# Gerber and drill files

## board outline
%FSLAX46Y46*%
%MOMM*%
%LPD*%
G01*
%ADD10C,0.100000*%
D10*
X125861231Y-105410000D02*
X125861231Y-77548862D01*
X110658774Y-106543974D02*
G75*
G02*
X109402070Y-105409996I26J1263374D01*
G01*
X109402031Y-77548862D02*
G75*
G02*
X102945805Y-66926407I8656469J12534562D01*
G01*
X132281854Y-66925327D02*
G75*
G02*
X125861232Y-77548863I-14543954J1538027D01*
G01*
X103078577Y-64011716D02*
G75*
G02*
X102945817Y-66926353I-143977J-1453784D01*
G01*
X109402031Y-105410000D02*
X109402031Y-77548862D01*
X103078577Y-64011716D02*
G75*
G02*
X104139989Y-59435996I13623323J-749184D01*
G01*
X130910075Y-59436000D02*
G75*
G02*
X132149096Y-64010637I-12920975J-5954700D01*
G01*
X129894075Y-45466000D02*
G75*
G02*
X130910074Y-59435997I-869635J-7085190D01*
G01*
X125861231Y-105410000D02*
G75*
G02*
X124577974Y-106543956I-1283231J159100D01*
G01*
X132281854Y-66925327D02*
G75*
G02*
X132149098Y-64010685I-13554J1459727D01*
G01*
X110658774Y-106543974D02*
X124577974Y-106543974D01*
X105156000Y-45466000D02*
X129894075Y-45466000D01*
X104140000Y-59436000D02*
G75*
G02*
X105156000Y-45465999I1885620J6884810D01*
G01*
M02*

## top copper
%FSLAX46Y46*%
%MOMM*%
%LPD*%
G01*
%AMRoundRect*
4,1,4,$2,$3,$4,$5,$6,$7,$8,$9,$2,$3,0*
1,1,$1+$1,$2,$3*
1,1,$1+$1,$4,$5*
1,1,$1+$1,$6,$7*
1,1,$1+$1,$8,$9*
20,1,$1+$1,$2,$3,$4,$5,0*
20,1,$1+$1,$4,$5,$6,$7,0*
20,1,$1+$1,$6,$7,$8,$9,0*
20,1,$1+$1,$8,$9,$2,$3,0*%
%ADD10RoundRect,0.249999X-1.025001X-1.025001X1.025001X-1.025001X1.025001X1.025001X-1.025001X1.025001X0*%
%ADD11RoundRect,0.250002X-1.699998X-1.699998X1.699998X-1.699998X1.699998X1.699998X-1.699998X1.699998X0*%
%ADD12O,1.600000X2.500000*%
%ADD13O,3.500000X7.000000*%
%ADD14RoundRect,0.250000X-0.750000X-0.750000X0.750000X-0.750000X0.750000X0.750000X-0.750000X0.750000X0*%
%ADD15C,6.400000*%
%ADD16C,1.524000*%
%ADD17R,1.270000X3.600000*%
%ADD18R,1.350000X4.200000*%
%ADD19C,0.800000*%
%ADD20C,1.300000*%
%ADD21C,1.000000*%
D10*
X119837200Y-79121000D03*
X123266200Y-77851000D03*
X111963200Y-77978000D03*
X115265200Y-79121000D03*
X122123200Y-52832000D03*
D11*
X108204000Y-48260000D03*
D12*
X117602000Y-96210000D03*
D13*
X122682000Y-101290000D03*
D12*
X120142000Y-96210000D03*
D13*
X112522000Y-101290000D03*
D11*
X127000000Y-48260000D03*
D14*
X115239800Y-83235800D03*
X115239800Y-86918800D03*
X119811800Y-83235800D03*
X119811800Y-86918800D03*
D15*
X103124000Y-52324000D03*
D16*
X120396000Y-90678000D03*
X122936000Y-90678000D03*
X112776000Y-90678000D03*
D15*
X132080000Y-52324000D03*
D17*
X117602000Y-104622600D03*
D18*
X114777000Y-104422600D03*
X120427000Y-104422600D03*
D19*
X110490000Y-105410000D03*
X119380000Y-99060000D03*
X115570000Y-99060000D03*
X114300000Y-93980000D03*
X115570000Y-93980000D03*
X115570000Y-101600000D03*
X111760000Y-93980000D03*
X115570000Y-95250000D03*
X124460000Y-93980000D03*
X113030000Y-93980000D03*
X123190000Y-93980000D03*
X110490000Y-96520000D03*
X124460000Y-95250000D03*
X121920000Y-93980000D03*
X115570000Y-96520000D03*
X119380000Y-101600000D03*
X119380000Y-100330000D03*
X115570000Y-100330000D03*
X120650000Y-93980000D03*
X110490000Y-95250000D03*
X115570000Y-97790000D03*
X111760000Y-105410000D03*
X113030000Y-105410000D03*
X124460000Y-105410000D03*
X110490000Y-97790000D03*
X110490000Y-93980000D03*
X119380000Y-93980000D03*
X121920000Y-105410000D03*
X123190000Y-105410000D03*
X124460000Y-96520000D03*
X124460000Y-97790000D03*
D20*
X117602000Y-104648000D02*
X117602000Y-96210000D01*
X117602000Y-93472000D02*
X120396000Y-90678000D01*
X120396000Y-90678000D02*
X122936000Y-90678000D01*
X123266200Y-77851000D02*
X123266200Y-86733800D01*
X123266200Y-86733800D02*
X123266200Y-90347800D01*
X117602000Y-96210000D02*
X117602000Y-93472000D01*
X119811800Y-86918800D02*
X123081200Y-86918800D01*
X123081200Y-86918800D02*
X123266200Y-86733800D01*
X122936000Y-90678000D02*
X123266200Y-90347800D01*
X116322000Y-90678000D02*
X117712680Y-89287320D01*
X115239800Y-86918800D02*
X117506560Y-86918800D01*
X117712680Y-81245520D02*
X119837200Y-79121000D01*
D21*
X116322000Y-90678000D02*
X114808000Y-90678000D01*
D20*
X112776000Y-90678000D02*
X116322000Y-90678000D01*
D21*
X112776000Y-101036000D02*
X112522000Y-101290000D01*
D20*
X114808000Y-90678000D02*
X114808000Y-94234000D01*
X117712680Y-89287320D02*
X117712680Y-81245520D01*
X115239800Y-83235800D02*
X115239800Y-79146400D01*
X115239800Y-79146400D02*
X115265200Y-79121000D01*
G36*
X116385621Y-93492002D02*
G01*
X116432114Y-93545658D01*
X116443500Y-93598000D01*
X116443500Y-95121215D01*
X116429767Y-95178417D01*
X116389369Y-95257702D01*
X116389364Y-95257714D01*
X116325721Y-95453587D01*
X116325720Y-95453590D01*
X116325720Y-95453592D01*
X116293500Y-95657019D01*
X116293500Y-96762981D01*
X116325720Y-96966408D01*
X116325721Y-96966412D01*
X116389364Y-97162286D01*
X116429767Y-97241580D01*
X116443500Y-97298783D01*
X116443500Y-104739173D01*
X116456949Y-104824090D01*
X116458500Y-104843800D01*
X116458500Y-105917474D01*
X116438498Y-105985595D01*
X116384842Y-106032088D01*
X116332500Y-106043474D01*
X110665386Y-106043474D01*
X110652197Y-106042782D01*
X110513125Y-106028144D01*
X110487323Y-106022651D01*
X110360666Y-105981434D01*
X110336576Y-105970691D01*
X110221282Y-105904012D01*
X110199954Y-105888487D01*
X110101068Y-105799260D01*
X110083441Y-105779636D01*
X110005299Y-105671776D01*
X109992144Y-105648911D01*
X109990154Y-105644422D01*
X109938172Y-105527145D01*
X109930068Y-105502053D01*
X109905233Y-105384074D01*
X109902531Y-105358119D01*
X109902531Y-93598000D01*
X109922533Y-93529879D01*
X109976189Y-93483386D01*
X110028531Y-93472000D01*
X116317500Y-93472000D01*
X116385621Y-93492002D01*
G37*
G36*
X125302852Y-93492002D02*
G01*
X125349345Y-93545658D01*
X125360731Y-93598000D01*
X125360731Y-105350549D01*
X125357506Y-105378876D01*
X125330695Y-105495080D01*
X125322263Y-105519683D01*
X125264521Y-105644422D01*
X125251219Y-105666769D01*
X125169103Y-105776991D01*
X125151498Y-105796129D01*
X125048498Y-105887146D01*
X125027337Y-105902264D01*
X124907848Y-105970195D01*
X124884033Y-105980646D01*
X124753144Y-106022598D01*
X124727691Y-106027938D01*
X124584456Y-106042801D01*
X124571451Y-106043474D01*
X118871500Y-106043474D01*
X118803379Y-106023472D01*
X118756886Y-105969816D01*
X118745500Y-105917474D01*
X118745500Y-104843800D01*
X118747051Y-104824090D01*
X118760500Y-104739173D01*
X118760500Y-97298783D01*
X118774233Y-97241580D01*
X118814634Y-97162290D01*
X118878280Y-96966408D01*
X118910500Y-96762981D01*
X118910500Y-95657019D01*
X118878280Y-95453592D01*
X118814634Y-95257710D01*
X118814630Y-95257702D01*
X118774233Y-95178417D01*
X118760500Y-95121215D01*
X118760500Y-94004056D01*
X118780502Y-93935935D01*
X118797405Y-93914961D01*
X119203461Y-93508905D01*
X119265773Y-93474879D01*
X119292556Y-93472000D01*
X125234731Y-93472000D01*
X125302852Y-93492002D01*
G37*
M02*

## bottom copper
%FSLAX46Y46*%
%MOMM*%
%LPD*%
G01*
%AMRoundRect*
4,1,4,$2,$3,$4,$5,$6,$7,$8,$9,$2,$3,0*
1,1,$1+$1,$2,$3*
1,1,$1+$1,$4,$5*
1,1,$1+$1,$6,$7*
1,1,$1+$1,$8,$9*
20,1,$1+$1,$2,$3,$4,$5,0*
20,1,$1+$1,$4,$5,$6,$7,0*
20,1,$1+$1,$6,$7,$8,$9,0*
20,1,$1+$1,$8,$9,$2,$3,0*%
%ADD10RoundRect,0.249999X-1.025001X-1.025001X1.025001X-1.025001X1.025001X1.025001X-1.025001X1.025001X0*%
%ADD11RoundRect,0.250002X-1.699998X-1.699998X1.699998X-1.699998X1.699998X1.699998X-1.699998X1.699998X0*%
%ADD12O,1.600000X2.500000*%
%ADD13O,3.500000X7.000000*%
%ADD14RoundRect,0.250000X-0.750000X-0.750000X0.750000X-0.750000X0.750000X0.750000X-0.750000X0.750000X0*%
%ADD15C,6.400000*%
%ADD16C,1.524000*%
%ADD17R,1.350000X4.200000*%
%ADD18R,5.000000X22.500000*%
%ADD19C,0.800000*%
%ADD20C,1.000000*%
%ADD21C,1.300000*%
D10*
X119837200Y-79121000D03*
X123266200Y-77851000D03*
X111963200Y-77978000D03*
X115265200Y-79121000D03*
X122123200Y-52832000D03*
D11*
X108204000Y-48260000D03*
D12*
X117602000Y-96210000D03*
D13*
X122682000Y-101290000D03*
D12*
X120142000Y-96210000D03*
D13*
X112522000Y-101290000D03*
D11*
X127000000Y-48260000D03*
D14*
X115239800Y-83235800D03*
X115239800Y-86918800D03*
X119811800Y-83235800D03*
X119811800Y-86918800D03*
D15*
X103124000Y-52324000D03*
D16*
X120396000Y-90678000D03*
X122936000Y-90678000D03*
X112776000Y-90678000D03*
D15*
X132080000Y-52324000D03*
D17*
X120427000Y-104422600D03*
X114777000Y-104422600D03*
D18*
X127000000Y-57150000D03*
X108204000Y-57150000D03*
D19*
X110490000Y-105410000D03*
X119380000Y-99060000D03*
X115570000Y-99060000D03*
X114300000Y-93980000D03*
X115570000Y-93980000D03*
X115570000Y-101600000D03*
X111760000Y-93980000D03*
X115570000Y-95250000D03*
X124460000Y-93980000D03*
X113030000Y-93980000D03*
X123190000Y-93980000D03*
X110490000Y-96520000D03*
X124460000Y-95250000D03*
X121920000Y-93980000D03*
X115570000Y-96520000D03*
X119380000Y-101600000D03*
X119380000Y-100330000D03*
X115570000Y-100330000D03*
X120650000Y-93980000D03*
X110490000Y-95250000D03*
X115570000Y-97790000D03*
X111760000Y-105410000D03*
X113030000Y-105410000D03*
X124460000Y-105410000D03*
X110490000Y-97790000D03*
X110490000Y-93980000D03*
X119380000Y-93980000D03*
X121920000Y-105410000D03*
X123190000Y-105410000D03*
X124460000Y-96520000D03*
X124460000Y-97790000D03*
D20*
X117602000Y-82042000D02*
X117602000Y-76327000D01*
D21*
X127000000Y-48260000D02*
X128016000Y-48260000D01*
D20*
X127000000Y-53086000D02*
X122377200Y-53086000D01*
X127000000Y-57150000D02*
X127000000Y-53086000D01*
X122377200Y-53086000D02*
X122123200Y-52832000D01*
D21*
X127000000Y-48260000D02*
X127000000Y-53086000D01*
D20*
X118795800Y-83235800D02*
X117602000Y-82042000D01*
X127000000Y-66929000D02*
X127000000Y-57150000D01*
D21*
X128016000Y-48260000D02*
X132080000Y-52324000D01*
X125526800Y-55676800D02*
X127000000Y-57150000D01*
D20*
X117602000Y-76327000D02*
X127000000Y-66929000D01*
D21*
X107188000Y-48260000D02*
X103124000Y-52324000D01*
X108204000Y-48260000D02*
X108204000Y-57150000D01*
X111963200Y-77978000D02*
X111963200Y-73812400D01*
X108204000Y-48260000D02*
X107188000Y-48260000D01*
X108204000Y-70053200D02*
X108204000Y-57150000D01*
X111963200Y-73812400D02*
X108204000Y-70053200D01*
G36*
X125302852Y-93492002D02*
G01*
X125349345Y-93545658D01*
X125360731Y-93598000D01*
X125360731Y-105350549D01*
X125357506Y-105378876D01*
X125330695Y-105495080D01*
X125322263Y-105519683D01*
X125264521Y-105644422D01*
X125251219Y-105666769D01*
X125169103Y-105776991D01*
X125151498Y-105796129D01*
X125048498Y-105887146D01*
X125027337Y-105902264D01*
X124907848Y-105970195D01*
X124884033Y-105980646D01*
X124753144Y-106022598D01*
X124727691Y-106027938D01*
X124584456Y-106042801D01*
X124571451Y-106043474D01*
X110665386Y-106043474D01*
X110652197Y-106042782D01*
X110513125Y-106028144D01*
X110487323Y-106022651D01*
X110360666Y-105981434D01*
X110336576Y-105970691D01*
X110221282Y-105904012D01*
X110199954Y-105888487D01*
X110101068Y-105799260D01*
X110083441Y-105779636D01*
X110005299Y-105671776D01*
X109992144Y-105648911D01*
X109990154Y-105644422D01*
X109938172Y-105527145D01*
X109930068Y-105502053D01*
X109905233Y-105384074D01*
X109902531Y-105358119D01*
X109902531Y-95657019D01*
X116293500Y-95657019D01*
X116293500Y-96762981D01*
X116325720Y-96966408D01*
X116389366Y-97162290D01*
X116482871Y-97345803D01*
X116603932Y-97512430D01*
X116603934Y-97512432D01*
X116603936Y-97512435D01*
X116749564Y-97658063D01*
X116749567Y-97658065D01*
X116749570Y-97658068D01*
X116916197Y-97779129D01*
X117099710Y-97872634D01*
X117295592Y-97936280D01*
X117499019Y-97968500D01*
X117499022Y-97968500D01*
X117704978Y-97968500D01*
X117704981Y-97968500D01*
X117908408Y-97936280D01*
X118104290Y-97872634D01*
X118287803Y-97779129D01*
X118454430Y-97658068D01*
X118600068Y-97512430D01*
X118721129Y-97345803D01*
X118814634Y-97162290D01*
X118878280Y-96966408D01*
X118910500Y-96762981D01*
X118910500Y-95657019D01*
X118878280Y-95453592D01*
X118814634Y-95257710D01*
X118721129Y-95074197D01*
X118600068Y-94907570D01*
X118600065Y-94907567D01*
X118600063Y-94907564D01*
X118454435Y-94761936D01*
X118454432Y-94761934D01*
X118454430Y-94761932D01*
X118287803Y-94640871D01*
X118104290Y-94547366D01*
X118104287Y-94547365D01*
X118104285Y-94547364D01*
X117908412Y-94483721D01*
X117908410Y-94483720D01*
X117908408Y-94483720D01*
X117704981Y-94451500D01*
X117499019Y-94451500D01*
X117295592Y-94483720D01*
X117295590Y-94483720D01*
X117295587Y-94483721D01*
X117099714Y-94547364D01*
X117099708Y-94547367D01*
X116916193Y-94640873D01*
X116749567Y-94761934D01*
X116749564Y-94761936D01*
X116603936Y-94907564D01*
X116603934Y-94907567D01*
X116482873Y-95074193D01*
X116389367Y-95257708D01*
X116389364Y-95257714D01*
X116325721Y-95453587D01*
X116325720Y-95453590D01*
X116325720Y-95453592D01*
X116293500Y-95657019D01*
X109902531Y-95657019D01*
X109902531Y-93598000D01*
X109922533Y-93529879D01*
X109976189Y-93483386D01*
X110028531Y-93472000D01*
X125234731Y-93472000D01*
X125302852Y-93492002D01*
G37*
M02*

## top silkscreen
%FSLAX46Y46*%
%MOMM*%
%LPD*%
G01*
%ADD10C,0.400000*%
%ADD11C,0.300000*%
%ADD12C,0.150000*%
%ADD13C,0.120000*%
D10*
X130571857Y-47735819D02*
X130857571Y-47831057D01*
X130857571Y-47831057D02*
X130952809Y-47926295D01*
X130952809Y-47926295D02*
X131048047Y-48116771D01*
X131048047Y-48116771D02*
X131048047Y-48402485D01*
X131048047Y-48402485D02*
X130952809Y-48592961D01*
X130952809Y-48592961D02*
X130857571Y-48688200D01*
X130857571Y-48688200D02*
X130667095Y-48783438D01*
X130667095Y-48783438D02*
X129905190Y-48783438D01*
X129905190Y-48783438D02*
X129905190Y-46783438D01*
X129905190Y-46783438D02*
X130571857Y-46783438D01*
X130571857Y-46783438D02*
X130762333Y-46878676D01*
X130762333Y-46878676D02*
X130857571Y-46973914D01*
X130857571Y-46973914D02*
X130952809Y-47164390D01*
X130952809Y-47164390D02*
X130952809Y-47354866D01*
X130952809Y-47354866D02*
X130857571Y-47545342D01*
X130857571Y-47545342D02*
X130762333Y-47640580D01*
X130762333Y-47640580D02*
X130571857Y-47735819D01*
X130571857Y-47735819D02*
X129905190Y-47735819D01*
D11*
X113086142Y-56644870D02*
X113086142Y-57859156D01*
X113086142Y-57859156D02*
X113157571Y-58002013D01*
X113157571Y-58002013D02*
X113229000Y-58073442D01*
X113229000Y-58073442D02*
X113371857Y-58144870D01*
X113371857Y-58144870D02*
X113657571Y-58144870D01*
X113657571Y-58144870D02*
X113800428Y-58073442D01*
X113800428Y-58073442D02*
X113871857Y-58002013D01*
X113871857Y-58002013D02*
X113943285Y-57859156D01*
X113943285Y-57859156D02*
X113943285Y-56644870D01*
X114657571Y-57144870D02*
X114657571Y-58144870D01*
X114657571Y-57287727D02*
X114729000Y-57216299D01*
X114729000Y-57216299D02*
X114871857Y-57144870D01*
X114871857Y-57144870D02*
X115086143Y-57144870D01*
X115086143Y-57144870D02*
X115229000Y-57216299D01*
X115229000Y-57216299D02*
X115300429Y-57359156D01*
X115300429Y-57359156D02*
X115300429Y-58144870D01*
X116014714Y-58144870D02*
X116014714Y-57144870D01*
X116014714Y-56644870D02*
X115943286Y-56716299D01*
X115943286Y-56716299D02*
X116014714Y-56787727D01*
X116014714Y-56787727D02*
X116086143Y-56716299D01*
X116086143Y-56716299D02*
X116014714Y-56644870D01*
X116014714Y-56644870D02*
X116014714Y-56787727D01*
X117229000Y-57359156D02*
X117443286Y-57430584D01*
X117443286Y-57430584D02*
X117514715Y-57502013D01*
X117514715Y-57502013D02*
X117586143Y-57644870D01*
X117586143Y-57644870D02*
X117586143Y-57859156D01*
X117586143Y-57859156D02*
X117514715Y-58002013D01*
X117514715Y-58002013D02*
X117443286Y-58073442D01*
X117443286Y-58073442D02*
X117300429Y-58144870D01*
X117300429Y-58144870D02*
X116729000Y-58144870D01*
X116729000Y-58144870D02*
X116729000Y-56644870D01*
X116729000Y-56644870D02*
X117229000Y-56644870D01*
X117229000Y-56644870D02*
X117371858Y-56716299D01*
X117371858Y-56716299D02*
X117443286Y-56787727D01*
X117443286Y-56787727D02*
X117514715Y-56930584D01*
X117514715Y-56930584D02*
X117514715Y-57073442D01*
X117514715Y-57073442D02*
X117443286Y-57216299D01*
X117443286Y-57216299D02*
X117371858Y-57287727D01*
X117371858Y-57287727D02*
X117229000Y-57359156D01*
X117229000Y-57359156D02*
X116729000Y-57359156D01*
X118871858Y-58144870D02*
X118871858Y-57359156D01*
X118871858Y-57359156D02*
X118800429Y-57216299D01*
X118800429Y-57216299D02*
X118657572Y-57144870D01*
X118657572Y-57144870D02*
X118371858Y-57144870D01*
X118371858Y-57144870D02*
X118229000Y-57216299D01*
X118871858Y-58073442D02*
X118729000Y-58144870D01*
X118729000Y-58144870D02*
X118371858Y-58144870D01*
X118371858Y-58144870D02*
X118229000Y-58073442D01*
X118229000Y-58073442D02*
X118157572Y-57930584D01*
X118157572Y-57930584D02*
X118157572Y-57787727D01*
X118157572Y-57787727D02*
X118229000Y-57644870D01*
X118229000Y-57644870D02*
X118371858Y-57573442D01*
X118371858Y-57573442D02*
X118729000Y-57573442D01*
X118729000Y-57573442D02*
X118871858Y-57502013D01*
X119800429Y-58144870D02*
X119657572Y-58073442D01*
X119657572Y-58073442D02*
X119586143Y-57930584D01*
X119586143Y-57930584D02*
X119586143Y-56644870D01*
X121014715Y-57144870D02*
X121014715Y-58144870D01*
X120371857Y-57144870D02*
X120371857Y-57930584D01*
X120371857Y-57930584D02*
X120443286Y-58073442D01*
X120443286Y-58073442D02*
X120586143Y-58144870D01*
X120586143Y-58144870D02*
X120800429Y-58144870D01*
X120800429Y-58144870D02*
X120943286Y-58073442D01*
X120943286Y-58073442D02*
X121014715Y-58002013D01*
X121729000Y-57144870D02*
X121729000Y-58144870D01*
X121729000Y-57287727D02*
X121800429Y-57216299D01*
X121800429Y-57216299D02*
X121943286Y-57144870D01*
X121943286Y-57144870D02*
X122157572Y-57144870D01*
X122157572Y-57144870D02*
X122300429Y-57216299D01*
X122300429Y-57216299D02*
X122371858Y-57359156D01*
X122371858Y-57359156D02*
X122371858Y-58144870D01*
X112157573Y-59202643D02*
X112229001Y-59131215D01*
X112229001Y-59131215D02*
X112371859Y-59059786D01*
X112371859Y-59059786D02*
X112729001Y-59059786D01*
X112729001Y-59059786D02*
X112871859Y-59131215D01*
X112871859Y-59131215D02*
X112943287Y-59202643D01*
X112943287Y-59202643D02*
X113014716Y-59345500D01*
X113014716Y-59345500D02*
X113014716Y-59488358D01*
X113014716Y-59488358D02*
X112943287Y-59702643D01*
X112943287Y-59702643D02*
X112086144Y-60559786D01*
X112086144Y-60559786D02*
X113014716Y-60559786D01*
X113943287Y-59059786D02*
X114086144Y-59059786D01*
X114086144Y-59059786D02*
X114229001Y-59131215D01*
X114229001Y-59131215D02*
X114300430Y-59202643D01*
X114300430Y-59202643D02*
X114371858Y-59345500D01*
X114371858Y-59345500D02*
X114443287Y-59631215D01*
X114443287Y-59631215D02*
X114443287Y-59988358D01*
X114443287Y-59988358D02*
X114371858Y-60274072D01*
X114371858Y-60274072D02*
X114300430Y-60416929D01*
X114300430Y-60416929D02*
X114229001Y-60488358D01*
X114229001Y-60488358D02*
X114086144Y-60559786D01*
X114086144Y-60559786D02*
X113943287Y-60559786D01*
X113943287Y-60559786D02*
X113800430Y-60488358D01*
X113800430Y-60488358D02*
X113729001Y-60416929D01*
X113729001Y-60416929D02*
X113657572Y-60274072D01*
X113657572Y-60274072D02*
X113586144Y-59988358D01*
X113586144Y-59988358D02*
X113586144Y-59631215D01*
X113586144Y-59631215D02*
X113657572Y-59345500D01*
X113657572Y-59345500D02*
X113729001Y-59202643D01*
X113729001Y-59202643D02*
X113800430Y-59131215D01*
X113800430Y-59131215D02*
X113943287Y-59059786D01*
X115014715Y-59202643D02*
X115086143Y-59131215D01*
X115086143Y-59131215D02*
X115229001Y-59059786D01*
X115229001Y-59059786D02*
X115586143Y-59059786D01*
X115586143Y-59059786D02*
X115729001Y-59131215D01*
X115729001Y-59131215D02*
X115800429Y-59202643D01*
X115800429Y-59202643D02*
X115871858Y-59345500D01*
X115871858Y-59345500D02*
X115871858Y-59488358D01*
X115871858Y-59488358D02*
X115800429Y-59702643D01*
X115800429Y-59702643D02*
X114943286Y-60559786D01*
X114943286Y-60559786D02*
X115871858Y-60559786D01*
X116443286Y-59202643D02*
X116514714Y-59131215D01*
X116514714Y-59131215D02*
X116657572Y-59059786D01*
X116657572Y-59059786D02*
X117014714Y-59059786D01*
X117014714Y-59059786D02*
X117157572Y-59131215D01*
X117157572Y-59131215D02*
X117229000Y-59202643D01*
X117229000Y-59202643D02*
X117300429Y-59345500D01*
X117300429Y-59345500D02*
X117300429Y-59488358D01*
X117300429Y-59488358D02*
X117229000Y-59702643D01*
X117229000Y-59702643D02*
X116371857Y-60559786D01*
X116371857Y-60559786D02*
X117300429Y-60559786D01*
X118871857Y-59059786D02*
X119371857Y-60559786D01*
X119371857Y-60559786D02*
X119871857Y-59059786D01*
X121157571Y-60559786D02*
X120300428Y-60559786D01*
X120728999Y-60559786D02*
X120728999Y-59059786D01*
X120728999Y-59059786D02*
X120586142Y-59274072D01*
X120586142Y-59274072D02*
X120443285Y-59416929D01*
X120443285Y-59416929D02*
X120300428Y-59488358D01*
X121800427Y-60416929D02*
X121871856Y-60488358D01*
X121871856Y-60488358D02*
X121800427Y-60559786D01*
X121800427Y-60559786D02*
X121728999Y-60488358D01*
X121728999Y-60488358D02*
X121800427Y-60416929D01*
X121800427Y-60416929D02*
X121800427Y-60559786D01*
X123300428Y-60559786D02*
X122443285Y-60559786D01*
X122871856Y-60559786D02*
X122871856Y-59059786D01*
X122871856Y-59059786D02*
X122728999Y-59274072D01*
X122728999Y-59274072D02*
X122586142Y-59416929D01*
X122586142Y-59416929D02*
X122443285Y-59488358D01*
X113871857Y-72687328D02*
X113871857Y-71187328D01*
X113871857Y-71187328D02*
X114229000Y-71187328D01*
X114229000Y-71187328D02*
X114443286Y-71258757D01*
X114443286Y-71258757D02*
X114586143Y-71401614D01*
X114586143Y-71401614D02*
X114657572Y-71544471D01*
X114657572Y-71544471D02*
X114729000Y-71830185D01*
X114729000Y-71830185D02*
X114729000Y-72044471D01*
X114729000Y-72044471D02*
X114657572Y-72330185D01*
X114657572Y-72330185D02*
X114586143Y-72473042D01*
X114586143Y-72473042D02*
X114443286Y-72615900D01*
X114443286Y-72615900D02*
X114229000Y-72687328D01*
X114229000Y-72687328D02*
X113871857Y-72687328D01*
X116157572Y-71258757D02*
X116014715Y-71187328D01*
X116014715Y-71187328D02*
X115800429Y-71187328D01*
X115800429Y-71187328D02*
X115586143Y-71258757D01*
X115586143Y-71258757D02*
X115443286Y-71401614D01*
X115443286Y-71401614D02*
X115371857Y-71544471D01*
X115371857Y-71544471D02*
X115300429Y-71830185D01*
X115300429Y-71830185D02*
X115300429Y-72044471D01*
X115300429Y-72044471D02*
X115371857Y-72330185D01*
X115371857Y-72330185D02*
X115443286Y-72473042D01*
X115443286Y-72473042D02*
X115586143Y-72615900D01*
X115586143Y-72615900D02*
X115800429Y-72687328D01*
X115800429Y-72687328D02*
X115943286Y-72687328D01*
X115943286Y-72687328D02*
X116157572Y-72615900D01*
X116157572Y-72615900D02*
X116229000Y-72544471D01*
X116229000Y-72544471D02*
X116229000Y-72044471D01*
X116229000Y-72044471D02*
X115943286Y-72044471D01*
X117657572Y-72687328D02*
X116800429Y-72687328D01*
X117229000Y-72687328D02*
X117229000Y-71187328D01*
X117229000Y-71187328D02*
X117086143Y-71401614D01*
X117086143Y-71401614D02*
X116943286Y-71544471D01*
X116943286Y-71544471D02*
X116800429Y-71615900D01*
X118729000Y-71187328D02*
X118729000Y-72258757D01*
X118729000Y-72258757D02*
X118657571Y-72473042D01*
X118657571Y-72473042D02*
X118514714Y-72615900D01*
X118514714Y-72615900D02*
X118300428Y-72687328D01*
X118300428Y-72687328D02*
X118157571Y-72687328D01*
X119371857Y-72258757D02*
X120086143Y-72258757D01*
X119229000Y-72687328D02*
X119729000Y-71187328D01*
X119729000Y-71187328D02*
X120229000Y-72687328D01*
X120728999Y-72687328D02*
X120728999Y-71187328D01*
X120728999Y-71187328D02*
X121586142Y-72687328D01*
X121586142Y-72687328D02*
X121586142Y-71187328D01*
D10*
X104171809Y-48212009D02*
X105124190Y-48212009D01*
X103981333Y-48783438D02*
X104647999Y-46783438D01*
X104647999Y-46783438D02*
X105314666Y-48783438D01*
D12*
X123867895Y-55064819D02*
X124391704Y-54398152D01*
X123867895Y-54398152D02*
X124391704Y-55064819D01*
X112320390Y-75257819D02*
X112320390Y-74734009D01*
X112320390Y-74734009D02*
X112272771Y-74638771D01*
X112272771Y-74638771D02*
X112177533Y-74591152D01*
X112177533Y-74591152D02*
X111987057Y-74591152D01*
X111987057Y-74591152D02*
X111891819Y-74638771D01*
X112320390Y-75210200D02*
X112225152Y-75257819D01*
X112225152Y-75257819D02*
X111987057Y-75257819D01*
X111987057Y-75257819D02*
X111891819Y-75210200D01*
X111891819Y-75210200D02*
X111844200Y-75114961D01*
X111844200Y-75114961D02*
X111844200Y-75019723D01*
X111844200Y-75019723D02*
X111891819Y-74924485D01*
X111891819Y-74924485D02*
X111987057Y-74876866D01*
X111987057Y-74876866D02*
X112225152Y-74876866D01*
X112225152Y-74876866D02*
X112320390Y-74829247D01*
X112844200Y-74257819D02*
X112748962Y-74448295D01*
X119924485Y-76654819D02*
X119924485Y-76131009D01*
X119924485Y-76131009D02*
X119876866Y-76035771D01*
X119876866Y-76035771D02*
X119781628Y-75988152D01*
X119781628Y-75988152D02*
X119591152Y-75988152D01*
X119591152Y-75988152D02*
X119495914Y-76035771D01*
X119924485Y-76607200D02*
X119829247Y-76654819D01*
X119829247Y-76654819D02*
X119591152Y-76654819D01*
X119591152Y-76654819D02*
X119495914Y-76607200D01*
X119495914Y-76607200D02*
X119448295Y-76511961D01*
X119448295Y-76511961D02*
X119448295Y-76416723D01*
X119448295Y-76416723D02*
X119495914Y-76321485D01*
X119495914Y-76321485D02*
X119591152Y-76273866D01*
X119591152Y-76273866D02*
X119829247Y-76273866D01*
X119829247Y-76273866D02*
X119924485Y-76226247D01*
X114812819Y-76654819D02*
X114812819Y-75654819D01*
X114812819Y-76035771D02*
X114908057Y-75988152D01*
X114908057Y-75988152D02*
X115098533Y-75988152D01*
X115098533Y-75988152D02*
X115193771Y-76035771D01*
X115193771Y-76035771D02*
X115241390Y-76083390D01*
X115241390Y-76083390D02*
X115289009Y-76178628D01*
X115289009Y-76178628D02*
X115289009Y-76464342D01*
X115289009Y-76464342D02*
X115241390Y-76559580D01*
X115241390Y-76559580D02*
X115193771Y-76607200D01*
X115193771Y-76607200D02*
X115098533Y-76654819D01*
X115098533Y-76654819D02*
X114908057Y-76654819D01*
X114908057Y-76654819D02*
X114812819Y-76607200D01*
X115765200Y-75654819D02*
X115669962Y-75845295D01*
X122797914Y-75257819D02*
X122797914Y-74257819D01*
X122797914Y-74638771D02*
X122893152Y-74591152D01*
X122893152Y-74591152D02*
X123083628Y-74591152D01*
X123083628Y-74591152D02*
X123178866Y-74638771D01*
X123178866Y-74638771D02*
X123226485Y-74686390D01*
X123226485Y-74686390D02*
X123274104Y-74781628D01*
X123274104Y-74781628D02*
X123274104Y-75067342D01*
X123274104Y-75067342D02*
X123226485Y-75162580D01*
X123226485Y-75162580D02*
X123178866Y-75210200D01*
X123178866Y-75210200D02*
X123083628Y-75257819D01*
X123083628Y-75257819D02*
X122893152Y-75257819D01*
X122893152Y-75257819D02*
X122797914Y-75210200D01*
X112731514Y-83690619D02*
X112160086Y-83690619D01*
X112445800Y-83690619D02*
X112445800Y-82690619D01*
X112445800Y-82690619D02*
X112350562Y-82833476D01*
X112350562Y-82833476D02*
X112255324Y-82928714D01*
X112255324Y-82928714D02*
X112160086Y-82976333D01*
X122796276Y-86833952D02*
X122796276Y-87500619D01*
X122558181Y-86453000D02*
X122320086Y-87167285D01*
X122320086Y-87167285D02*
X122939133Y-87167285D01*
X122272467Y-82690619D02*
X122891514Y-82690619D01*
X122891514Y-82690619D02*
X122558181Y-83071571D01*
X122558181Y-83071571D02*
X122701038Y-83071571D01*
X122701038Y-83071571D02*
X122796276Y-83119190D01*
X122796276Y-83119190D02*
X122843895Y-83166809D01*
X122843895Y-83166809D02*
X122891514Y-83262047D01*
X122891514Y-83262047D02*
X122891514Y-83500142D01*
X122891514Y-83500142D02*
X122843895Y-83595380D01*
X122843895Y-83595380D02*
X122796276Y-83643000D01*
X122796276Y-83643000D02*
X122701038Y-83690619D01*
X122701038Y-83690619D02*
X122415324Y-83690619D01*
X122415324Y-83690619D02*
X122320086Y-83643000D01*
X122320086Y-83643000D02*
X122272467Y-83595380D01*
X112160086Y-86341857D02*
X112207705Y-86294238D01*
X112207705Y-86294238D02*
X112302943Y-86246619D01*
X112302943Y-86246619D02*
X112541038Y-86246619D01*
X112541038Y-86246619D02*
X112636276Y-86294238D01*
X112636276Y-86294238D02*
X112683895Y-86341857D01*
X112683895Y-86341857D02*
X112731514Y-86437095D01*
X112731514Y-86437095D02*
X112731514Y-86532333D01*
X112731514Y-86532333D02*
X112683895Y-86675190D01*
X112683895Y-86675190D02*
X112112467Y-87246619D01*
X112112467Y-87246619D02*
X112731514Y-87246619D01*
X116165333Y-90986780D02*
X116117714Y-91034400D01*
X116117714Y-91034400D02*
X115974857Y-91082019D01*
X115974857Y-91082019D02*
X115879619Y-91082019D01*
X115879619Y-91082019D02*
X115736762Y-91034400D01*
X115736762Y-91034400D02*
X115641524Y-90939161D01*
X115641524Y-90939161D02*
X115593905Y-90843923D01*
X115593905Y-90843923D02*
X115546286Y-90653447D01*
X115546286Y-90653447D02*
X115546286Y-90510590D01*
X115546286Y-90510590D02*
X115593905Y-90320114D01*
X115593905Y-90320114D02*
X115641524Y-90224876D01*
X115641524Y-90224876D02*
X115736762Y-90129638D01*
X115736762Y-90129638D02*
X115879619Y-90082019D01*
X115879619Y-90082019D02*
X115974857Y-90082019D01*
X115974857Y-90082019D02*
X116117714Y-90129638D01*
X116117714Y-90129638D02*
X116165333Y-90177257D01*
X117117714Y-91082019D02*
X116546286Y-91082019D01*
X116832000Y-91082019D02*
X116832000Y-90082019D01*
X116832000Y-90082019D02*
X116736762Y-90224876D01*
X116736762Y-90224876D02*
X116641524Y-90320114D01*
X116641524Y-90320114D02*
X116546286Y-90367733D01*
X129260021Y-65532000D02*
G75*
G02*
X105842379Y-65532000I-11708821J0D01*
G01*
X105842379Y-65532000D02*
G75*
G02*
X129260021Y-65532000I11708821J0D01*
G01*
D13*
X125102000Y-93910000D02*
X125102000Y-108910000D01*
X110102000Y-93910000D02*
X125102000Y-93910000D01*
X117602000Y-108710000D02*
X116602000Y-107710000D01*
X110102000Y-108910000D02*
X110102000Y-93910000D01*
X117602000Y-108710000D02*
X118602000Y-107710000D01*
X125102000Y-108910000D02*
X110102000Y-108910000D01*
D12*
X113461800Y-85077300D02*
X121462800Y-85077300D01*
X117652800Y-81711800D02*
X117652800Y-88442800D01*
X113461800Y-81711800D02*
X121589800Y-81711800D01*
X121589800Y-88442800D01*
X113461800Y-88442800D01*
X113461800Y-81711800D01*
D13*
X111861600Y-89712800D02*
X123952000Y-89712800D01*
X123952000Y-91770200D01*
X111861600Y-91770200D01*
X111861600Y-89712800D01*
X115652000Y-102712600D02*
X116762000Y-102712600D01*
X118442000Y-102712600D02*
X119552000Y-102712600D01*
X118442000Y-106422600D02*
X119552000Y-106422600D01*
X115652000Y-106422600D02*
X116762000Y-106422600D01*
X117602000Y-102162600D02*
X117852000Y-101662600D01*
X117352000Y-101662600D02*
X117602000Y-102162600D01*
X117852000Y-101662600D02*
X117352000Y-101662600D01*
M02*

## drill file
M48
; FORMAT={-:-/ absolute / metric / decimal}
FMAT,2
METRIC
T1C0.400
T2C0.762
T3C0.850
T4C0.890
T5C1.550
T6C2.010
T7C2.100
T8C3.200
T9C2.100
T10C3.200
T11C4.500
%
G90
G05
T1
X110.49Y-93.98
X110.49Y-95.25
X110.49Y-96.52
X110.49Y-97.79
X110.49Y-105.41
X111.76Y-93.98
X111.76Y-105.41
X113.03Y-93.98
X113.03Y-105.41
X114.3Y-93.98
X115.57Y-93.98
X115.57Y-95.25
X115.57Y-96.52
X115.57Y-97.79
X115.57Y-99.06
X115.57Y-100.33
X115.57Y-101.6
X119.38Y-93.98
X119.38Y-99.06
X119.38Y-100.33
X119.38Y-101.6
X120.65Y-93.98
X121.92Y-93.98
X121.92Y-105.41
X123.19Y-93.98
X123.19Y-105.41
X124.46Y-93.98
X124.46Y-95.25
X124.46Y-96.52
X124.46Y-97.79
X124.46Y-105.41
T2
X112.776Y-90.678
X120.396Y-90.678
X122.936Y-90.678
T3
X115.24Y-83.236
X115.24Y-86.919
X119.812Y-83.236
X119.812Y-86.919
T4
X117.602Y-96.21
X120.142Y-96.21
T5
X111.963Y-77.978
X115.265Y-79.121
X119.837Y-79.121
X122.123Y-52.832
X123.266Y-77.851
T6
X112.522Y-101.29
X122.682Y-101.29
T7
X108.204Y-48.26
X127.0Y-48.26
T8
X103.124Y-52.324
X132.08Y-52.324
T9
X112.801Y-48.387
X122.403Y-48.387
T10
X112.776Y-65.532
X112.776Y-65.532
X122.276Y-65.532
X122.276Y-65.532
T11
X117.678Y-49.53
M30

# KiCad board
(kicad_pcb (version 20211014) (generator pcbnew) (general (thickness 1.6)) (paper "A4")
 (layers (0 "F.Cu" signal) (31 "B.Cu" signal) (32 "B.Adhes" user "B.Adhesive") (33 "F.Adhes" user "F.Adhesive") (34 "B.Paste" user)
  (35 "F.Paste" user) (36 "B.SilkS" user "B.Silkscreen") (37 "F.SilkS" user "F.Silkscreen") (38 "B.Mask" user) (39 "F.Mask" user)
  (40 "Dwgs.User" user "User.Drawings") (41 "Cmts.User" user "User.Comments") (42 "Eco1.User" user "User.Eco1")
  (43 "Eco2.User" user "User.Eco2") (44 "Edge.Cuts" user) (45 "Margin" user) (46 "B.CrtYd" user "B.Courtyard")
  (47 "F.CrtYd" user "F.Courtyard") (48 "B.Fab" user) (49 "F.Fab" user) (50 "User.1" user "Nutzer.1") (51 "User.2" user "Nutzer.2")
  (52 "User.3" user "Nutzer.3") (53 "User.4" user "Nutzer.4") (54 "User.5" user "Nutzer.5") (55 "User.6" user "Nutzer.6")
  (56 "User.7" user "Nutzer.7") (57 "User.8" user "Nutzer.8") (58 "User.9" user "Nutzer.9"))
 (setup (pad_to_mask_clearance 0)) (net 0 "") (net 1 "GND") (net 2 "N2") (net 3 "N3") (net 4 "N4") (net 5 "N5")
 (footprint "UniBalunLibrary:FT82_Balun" (layer "F.Cu") (at 117.602 65.532)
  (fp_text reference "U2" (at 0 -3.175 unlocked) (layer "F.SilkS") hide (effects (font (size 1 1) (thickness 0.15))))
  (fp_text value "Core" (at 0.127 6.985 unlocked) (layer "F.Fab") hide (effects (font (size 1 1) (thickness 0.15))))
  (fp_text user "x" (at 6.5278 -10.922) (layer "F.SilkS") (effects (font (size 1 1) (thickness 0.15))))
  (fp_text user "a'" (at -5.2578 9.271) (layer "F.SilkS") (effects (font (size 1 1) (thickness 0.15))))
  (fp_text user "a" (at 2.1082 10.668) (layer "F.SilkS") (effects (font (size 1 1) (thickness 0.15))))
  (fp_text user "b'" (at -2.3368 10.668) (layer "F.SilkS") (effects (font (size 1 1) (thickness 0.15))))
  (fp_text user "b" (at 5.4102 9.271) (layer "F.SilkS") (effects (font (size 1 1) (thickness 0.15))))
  (fp_circle (center -0.0508 0) (end -2.5908 11.43) (layer "F.SilkS") (width 0.15) (fill none))
  (pad "" np_thru_hole circle (at 4.6736 0) (size 3.2 3.2) (drill 3.2) (layers *.Cu *.Mask))
  (pad "" np_thru_hole circle (at -4.826 0) (size 3.2 3.2) (drill 3.2) (layers *.Cu *.Mask))
  (pad "" np_thru_hole circle (at -4.826 0) (size 3.2 3.2) (drill 3.2) (layers *.Cu *.Mask))
  (pad "" np_thru_hole circle (at 4.6736 0) (size 3.2 3.2) (drill 3.2) (layers *.Cu *.Mask))
  (pad "1" thru_hole roundrect (at 2.2352 13.589) (size 2.55 2.55) (drill 1.55) (layers *.Cu *.Mask) (roundrect_rratio 0.098039)
   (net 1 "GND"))
  (pad "2" thru_hole roundrect (at 5.6642 12.319) (size 2.55 2.55) (drill 1.55) (layers *.Cu *.Mask) (roundrect_rratio 0.098039)
   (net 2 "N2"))
  (pad "3" thru_hole roundrect (at -5.6388 12.446) (size 2.55 2.55) (drill 1.55) (layers *.Cu *.Mask) (roundrect_rratio 0.098039)
   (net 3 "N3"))
  (pad "4" thru_hole roundrect (at -2.3368 13.589) (size 2.55 2.55) (drill 1.55) (layers *.Cu *.Mask) (roundrect_rratio 0.098039)
   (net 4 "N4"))
  (pad "5" thru_hole roundrect (at 4.5212 -12.7) (size 2.55 2.55) (drill 1.55) (layers *.Cu *.Mask) (roundrect_rratio 0.098039) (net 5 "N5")))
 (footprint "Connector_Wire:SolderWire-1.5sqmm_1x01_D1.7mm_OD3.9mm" (layer "F.Cu") (at 108.204 48.26)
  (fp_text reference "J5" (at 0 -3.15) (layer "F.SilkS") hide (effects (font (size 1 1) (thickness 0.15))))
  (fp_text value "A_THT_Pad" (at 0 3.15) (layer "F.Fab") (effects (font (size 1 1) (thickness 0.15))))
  (pad "1" thru_hole roundrect (at 0 0) (size 3.9 3.9) (drill 2.1) (layers *.Cu *.Mask) (roundrect_rratio 0.064103) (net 3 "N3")))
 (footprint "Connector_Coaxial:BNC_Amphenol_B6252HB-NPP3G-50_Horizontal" (layer "F.Cu") (at 117.602 96.21 180)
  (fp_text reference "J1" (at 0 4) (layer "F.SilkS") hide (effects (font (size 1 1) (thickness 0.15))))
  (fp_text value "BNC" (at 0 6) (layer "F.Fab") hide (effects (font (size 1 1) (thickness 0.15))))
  (fp_line (start -7.5 2.3) (end -7.5 -12.7) (layer "F.SilkS") (width 0.12))
  (fp_line (start 7.5 2.3) (end -7.5 2.3) (layer "F.SilkS") (width 0.12))
  (fp_line (start 0 -12.5) (end 1 -11.5) (layer "F.SilkS") (width 0.12))
  (fp_line (start 7.5 -12.7) (end 7.5 2.3) (layer "F.SilkS") (width 0.12))
  (fp_line (start 0 -12.5) (end -1 -11.5) (layer "F.SilkS") (width 0.12))
  (fp_line (start -7.5 -12.7) (end 7.5 -12.7) (layer "F.SilkS") (width 0.12))
  (pad "1" thru_hole oval (at 0 0 180) (size 1.6 2.5) (drill 0.89) (layers *.Cu *.Mask) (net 2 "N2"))
  (pad "2" thru_hole oval (at -5.08 -5.08 180) (size 3.5 7) (drill 2.01) (layers *.Cu *.Mask) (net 1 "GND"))
  (pad "2" thru_hole oval (at -2.54 0 180) (size 1.6 2.5) (drill 0.89) (layers *.Cu *.Mask) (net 1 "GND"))
  (pad "2" thru_hole oval (at 5.08 -5.08 180) (size 3.5 7) (drill 2.01) (layers *.Cu *.Mask) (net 1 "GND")))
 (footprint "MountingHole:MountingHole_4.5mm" (layer "F.Cu") (at 117.6782 49.53)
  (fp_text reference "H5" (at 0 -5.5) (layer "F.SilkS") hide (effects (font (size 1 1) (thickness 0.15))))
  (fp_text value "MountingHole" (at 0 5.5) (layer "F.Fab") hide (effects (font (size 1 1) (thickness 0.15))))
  (pad "" np_thru_hole circle (at 0 0) (size 4.5 4.5) (drill 4.5) (layers *.Cu *.Mask)))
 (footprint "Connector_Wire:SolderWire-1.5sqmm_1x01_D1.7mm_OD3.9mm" (layer "F.Cu") (at 127 48.26)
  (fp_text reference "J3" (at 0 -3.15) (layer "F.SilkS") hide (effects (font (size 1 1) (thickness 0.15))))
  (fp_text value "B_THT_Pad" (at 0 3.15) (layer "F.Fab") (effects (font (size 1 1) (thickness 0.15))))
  (pad "1" thru_hole roundrect (at 0 0) (size 3.9 3.9) (drill 2.1) (layers *.Cu *.Mask) (roundrect_rratio 0.064103) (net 5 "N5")))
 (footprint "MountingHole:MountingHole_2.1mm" (layer "F.Cu") (at 112.8014 48.387)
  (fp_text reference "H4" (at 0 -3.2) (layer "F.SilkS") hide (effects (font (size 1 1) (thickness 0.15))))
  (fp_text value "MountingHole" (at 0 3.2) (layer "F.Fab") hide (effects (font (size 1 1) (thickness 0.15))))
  (pad "" np_thru_hole circle (at 0 0) (size 2.1 2.1) (drill 2.1) (layers *.Cu *.Mask)))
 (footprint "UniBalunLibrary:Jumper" (layer "F.Cu") (at 117.602 85.09)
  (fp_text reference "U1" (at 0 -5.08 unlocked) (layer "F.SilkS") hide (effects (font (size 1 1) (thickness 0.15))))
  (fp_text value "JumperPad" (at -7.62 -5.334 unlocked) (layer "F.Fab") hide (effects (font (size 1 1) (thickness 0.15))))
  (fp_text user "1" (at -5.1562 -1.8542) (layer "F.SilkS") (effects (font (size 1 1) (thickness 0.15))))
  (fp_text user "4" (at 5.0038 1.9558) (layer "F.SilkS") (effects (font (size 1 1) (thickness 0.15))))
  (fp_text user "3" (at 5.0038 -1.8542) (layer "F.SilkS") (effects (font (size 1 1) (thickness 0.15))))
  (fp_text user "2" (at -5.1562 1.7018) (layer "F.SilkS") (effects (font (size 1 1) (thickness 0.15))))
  (fp_line (start -4.1402 -0.0127) (end 3.8608 -0.0127) (layer "F.SilkS") (width 0.15))
  (fp_line (start 0.0508 -3.3782) (end 0.0508 3.3528) (layer "F.SilkS") (width 0.15))
  (fp_rect (start -4.1402 -3.3782) (end 3.9878 3.3528) (layer "F.SilkS") (width 0.15) (fill none))
  (pad "1" thru_hole roundrect (at -2.3622 -1.8542) (size 2 2) (drill 0.85) (layers *.Cu *.Mask) (roundrect_rratio 0.125) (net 4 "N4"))
  (pad "2" thru_hole roundrect (at -2.3622 1.8288) (size 2 2) (drill 0.85) (layers *.Cu *.Mask) (roundrect_rratio 0.125) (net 1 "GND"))
  (pad "3" thru_hole roundrect (at 2.2098 -1.8542) (size 2 2) (drill 0.85) (layers *.Cu *.Mask) (roundrect_rratio 0.125) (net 5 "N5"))
  (pad "4" thru_hole roundrect (at 2.2098 1.8288) (size 2 2) (drill 0.85) (layers *.Cu *.Mask) (roundrect_rratio 0.125) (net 2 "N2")))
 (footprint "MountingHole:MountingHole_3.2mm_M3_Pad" (layer "F.Cu") (at 103.124 52.324)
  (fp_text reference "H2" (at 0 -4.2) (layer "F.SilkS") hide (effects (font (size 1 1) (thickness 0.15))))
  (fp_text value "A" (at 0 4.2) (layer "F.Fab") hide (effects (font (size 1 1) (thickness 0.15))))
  (pad "1" thru_hole circle (at 0 0) (size 6.4 6.4) (drill 3.2) (layers *.Cu *.Mask) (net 3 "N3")))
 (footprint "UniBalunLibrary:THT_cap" (layer "F.Cu") (at 117.856 90.678 180)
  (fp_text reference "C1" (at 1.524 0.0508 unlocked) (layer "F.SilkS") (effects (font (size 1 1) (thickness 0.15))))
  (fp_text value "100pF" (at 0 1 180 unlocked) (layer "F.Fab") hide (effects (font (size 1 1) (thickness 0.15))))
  (fp_rect (start -6.096 -1.0922) (end 5.9944 0.9652) (layer "F.SilkS") (width 0.12) (fill none))
  (pad "1" thru_hole circle (at -2.54 0 180) (size 1.524 1.524) (drill 0.762) (layers *.Cu *.Mask) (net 2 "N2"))
  (pad "1" thru_hole circle (at -5.08 0 180) (size 1.524 1.524) (drill 0.762) (layers *.Cu *.Mask) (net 2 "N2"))
  (pad "2" thru_hole circle (at 5.08 0 180) (size 1.524 1.524) (drill 0.762) (layers *.Cu *.Mask) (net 1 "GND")))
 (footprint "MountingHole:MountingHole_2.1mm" (layer "F.Cu") (at 122.4026 48.387)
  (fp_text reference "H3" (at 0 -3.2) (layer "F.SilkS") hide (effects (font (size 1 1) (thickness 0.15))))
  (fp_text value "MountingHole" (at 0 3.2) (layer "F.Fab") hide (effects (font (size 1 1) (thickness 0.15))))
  (pad "" np_thru_hole circle (at 0 0) (size 2.1 2.1) (drill 2.1) (layers *.Cu *.Mask)))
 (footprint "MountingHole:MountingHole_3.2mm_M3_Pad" (layer "F.Cu") (at 132.08 52.324)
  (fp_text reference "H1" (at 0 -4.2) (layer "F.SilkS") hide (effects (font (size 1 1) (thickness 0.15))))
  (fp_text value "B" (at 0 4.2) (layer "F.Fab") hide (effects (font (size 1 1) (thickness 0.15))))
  (pad "1" thru_hole circle (at 0 0) (size 6.4 6.4) (drill 3.2) (layers *.Cu *.Mask) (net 5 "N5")))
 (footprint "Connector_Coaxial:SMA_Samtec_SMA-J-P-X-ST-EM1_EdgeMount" (layer "F.Cu") (at 117.602 104.4226)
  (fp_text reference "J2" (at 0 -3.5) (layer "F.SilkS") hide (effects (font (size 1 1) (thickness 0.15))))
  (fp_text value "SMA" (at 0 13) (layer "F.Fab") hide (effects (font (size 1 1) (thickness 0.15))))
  (fp_line (start -1.95 -1.71) (end -0.84 -1.71) (layer "F.SilkS") (width 0.12))
  (fp_line (start 0.84 -1.71) (end 1.95 -1.71) (layer "F.SilkS") (width 0.12))
  (fp_line (start 0.84 2) (end 1.95 2) (layer "F.SilkS") (width 0.12))
  (fp_line (start -1.95 2) (end -0.84 2) (layer "F.SilkS") (width 0.12))
  (fp_line (start 0 -2.26) (end 0.25 -2.76) (layer "F.SilkS") (width 0.12))
  (fp_line (start -0.25 -2.76) (end 0 -2.26) (layer "F.SilkS") (width 0.12))
  (fp_line (start 0.25 -2.76) (end -0.25 -2.76) (layer "F.SilkS") (width 0.12))
  (pad "1" smd rect (at 0 0.2) (size 1.27 3.6) (layers "F.Cu" "F.Paste" "F.Mask") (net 2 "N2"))
  (pad "2" smd rect (at 2.825 0) (size 1.35 4.2) (layers "B.Cu" "B.Paste" "B.Mask") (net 1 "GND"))
  (pad "2" smd rect (at -2.825 0) (size 1.35 4.2) (layers "B.Cu" "B.Paste" "B.Mask") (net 1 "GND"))
  (pad "2" smd rect (at -2.825 0) (size 1.35 4.2) (layers "F.Cu" "F.Paste" "F.Mask") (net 1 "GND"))
  (pad "2" smd rect (at 2.825 0) (size 1.35 4.2) (layers "F.Cu" "F.Paste" "F.Mask") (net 1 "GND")))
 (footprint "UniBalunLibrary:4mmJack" (layer "B.Cu") (at 127.254 56.896 90)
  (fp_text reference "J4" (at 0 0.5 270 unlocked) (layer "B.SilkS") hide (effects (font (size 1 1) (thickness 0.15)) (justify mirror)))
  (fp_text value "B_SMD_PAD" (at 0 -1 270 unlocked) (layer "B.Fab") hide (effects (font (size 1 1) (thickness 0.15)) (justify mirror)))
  (pad "1" smd rect (at -0.254 -0.254 90) (size 22.5 5) (layers "B.Cu" "B.Mask") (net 5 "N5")))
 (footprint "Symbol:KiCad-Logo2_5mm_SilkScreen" (layer "B.Cu") (at 117.729 58.547 180)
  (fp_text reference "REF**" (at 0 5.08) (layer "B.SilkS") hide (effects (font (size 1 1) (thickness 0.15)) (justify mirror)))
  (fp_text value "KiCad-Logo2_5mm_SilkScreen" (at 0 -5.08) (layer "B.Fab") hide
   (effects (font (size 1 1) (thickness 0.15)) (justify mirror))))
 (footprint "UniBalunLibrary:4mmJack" (layer "B.Cu") (at 108.458 56.896 90)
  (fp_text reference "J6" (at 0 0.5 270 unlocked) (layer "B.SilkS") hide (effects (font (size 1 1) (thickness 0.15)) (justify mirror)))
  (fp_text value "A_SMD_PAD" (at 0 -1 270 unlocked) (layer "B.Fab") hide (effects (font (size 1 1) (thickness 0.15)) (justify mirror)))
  (pad "1" smd rect (at -0.254 -0.254 90) (size 22.5 5) (layers "B.Cu" "B.Mask") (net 3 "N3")))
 (gr_line (start 125.861231 105.41) (end 125.861231 77.548862) (layer "Edge.Cuts") (width 0.1))
 (gr_arc (start 110.658774 106.543974) (mid 109.812413 106.218577) (end 109.402031 105.41) (layer "Edge.Cuts") (width 0.1))
 (gr_arc (start 109.402031 77.548862) (mid 105.04112 72.92614) (end 102.945817 66.926406) (layer "Edge.Cuts") (width 0.1))
 (gr_arc (start 132.281854 66.925327) (mid 130.254542 72.952072) (end 125.861231 77.548862) (layer "Edge.Cuts") (width 0.1))
 (gr_arc (start 103.078577 64.011716) (mid 104.394 65.532) (end 102.945817 66.926406) (layer "Edge.Cuts") (width 0.1))
 (gr_line (start 109.402031 105.41) (end 109.402031 77.548862) (layer "Edge.Cuts") (width 0.1))
 (gr_arc (start 103.078577 64.011716) (mid 103.410896 61.677837) (end 104.14 59.436) (layer "Edge.Cuts") (width 0.1))
 (gr_arc (start 130.910075 59.436) (mid 131.721418 61.671361) (end 132.149094 64.010637) (layer "Edge.Cuts") (width 0.1))
 (gr_arc (start 129.894075 45.466) (mid 136.144 52.033405) (end 130.910075 59.436) (layer "Edge.Cuts") (width 0.1))
 (gr_arc (start 125.861231 105.41) (mid 125.43422 106.219858) (end 124.577974 106.543974) (layer "Edge.Cuts") (width 0.1))
 (gr_arc (start 132.281854 66.925327) (mid 130.81 65.532) (end 132.149094 64.010637) (layer "Edge.Cuts") (width 0.1))
 (gr_line (start 110.658774 106.543974) (end 124.577974 106.543974) (layer "Edge.Cuts") (width 0.1))
 (gr_line (start 105.156 45.466) (end 129.894075 45.466) (layer "Edge.Cuts") (width 0.1))
 (gr_arc (start 104.14 59.436) (mid 98.906069 52.033405) (end 105.156 45.466) (layer "Edge.Cuts") (width 0.1))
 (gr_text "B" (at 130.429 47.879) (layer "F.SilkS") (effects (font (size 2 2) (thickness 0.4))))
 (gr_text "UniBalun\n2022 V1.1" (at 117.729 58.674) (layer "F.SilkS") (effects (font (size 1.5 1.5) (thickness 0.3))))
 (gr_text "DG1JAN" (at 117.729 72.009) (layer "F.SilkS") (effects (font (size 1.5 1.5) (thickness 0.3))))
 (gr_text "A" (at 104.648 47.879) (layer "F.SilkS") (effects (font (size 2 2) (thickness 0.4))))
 (segment (start 117.602 104.648) (end 117.602 96.21) (width 1.3) (layer "F.Cu") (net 2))
 (segment (start 117.602 93.472) (end 120.396 90.678) (width 1.3) (layer "F.Cu") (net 2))
 (segment (start 120.396 90.678) (end 122.936 90.678) (width 1.3) (layer "F.Cu") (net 2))
 (segment (start 123.2662 77.851) (end 123.2662 86.7338) (width 1.3) (layer "F.Cu") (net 2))
 (segment (start 123.2662 86.7338) (end 123.2662 90.3478) (width 1.3) (layer "F.Cu") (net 2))
 (segment (start 117.602 96.21) (end 117.602 93.472) (width 1.3) (layer "F.Cu") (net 2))
 (segment (start 119.8118 86.9188) (end 123.0812 86.9188) (width 1.3) (layer "F.Cu") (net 2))
 (segment (start 123.0812 86.9188) (end 123.2662 86.7338) (width 1.3) (layer "F.Cu") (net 2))
 (segment (start 122.936 90.678) (end 123.2662 90.3478) (width 1.3) (layer "F.Cu") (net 2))
 (segment (start 116.322 90.678) (end 117.71268 89.28732) (width 1.3) (layer "F.Cu") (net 1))
 (segment (start 115.2398 86.9188) (end 117.50656 86.9188) (width 1.3) (layer "F.Cu") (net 1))
 (segment (start 117.71268 81.24552) (end 119.8372 79.121) (width 1.3) (layer "F.Cu") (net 1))
 (segment (start 116.322 90.678) (end 114.808 90.678) (width 1) (layer "F.Cu") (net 1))
 (segment (start 112.776 90.678) (end 116.322 90.678) (width 1.3) (layer "F.Cu") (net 1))
 (segment (start 112.776 101.036) (end 112.522 101.29) (width 1) (layer "F.Cu") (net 1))
 (segment (start 114.808 90.678) (end 114.808 94.234) (width 1.3) (layer "F.Cu") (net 1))
 (segment (start 117.71268 89.28732) (end 117.71268 81.24552) (width 1.3) (layer "F.Cu") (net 1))
 (via (at 110.49 105.41) (size 0.8) (drill 0.4) (layers "F.Cu" "B.Cu") (free) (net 1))
 (via (at 119.38 99.06) (size 0.8) (drill 0.4) (layers "F.Cu" "B.Cu") (free) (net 1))
 (via (at 115.57 99.06) (size 0.8) (drill 0.4) (layers "F.Cu" "B.Cu") (free) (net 1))
 (via (at 114.3 93.98) (size 0.8) (drill 0.4) (layers "F.Cu" "B.Cu") (free) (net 1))
 (via (at 115.57 93.98) (size 0.8) (drill 0.4) (layers "F.Cu" "B.Cu") (free) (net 1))
 (via (at 115.57 101.6) (size 0.8) (drill 0.4) (layers "F.Cu" "B.Cu") (free) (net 1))
 (via (at 111.76 93.98) (size 0.8) (drill 0.4) (layers "F.Cu" "B.Cu") (free) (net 1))
 (via (at 115.57 95.25) (size 0.8) (drill 0.4) (layers "F.Cu" "B.Cu") (free) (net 1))
 (via (at 124.46 93.98) (size 0.8) (drill 0.4) (layers "F.Cu" "B.Cu") (free) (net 1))
 (via (at 113.03 93.98) (size 0.8) (drill 0.4) (layers "F.Cu" "B.Cu") (free) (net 1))
 (via (at 123.19 93.98) (size 0.8) (drill 0.4) (layers "F.Cu" "B.Cu") (free) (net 1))
 (via (at 110.49 96.52) (size 0.8) (drill 0.4) (layers "F.Cu" "B.Cu") (free) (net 1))
 (via (at 124.46 95.25) (size 0.8) (drill 0.4) (layers "F.Cu" "B.Cu") (free) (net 1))
 (via (at 121.92 93.98) (size 0.8) (drill 0.4) (layers "F.Cu" "B.Cu") (free) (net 1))
 (via (at 115.57 96.52) (size 0.8) (drill 0.4) (layers "F.Cu" "B.Cu") (free) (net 1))
 (via (at 119.38 101.6) (size 0.8) (drill 0.4) (layers "F.Cu" "B.Cu") (free) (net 1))
 (via (at 119.38 100.33) (size 0.8) (drill 0.4) (layers "F.Cu" "B.Cu") (free) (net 1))
 (via (at 115.57 100.33) (size 0.8) (drill 0.4) (layers "F.Cu" "B.Cu") (free) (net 1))
 (via (at 120.65 93.98) (size 0.8) (drill 0.4) (layers "F.Cu" "B.Cu") (free) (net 1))
 (via (at 110.49 95.25) (size 0.8) (drill 0.4) (layers "F.Cu" "B.Cu") (free) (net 1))
 (via (at 115.57 97.79) (size 0.8) (drill 0.4) (layers "F.Cu" "B.Cu") (free) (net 1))
 (via (at 111.76 105.41) (size 0.8) (drill 0.4) (layers "F.Cu" "B.Cu") (free) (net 1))
 (via (at 113.03 105.41) (size 0.8) (drill 0.4) (layers "F.Cu" "B.Cu") (free) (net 1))
 (via (at 124.46 105.41) (size 0.8) (drill 0.4) (layers "F.Cu" "B.Cu") (free) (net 1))
 (via (at 110.49 97.79) (size 0.8) (drill 0.4) (layers "F.Cu" "B.Cu") (free) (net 1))
 (via (at 110.49 93.98) (size 0.8) (drill 0.4) (layers "F.Cu" "B.Cu") (free) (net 1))
 (via (at 119.38 93.98) (size 0.8) (drill 0.4) (layers "F.Cu" "B.Cu") (free) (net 1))
 (via (at 121.92 105.41) (size 0.8) (drill 0.4) (layers "F.Cu" "B.Cu") (free) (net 1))
 (via (at 123.19 105.41) (size 0.8) (drill 0.4) (layers "F.Cu" "B.Cu") (free) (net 1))
 (via (at 124.46 96.52) (size 0.8) (drill 0.4) (layers "F.Cu" "B.Cu") (free) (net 1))
 (via (at 124.46 97.79) (size 0.8) (drill 0.4) (layers "F.Cu" "B.Cu") (free) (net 1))
 (segment (start 117.602 82.042) (end 117.602 76.327) (width 1) (layer "B.Cu") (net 5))
 (segment (start 127 48.26) (end 128.016 48.26) (width 1.3) (layer "B.Cu") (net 5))
 (segment (start 127 53.086) (end 122.3772 53.086) (width 1) (layer "B.Cu") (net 5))
 (segment (start 127 57.15) (end 127 53.086) (width 1) (layer "B.Cu") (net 5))
 (segment (start 122.3772 53.086) (end 122.1232 52.832) (width 1) (layer "B.Cu") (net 5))
 (segment (start 127 48.26) (end 127 53.086) (width 1.3) (layer "B.Cu") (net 5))
 (segment (start 118.7958 83.2358) (end 117.602 82.042) (width 1) (layer "B.Cu") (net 5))
 (segment (start 127 66.929) (end 127 57.15) (width 1) (layer "B.Cu") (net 5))
 (segment (start 128.016 48.26) (end 132.08 52.324) (width 1.3) (layer "B.Cu") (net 5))
 (segment (start 125.5268 55.6768) (end 127 57.15) (width 1.3) (layer "B.Cu") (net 5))
 (segment (start 117.602 76.327) (end 127 66.929) (width 1) (layer "B.Cu") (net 5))
 (segment (start 115.2398 83.2358) (end 115.2398 79.1464) (width 1.3) (layer "F.Cu") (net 4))
 (segment (start 115.2398 79.1464) (end 115.2652 79.121) (width 1.3) (layer "F.Cu") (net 4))
 (segment (start 107.188 48.26) (end 103.124 52.324) (width 1.3) (layer "B.Cu") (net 3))
 (segment (start 108.204 48.26) (end 108.204 57.15) (width 1.3) (layer "B.Cu") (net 3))
 (segment (start 111.9632 77.978) (end 111.9632 73.8124) (width 1.3) (layer "B.Cu") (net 3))
 (segment (start 108.204 48.26) (end 107.188 48.26) (width 1.3) (layer "B.Cu") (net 3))
 (segment (start 108.204 70.0532) (end 108.204 57.15) (width 1.3) (layer "B.Cu") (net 3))
 (segment (start 111.9632 73.8124) (end 108.204 70.0532) (width 1.3) (layer "B.Cu") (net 3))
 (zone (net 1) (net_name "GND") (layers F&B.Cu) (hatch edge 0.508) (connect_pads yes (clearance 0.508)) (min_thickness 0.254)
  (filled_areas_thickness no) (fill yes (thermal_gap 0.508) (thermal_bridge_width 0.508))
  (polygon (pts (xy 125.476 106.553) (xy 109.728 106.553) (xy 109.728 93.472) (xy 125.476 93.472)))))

